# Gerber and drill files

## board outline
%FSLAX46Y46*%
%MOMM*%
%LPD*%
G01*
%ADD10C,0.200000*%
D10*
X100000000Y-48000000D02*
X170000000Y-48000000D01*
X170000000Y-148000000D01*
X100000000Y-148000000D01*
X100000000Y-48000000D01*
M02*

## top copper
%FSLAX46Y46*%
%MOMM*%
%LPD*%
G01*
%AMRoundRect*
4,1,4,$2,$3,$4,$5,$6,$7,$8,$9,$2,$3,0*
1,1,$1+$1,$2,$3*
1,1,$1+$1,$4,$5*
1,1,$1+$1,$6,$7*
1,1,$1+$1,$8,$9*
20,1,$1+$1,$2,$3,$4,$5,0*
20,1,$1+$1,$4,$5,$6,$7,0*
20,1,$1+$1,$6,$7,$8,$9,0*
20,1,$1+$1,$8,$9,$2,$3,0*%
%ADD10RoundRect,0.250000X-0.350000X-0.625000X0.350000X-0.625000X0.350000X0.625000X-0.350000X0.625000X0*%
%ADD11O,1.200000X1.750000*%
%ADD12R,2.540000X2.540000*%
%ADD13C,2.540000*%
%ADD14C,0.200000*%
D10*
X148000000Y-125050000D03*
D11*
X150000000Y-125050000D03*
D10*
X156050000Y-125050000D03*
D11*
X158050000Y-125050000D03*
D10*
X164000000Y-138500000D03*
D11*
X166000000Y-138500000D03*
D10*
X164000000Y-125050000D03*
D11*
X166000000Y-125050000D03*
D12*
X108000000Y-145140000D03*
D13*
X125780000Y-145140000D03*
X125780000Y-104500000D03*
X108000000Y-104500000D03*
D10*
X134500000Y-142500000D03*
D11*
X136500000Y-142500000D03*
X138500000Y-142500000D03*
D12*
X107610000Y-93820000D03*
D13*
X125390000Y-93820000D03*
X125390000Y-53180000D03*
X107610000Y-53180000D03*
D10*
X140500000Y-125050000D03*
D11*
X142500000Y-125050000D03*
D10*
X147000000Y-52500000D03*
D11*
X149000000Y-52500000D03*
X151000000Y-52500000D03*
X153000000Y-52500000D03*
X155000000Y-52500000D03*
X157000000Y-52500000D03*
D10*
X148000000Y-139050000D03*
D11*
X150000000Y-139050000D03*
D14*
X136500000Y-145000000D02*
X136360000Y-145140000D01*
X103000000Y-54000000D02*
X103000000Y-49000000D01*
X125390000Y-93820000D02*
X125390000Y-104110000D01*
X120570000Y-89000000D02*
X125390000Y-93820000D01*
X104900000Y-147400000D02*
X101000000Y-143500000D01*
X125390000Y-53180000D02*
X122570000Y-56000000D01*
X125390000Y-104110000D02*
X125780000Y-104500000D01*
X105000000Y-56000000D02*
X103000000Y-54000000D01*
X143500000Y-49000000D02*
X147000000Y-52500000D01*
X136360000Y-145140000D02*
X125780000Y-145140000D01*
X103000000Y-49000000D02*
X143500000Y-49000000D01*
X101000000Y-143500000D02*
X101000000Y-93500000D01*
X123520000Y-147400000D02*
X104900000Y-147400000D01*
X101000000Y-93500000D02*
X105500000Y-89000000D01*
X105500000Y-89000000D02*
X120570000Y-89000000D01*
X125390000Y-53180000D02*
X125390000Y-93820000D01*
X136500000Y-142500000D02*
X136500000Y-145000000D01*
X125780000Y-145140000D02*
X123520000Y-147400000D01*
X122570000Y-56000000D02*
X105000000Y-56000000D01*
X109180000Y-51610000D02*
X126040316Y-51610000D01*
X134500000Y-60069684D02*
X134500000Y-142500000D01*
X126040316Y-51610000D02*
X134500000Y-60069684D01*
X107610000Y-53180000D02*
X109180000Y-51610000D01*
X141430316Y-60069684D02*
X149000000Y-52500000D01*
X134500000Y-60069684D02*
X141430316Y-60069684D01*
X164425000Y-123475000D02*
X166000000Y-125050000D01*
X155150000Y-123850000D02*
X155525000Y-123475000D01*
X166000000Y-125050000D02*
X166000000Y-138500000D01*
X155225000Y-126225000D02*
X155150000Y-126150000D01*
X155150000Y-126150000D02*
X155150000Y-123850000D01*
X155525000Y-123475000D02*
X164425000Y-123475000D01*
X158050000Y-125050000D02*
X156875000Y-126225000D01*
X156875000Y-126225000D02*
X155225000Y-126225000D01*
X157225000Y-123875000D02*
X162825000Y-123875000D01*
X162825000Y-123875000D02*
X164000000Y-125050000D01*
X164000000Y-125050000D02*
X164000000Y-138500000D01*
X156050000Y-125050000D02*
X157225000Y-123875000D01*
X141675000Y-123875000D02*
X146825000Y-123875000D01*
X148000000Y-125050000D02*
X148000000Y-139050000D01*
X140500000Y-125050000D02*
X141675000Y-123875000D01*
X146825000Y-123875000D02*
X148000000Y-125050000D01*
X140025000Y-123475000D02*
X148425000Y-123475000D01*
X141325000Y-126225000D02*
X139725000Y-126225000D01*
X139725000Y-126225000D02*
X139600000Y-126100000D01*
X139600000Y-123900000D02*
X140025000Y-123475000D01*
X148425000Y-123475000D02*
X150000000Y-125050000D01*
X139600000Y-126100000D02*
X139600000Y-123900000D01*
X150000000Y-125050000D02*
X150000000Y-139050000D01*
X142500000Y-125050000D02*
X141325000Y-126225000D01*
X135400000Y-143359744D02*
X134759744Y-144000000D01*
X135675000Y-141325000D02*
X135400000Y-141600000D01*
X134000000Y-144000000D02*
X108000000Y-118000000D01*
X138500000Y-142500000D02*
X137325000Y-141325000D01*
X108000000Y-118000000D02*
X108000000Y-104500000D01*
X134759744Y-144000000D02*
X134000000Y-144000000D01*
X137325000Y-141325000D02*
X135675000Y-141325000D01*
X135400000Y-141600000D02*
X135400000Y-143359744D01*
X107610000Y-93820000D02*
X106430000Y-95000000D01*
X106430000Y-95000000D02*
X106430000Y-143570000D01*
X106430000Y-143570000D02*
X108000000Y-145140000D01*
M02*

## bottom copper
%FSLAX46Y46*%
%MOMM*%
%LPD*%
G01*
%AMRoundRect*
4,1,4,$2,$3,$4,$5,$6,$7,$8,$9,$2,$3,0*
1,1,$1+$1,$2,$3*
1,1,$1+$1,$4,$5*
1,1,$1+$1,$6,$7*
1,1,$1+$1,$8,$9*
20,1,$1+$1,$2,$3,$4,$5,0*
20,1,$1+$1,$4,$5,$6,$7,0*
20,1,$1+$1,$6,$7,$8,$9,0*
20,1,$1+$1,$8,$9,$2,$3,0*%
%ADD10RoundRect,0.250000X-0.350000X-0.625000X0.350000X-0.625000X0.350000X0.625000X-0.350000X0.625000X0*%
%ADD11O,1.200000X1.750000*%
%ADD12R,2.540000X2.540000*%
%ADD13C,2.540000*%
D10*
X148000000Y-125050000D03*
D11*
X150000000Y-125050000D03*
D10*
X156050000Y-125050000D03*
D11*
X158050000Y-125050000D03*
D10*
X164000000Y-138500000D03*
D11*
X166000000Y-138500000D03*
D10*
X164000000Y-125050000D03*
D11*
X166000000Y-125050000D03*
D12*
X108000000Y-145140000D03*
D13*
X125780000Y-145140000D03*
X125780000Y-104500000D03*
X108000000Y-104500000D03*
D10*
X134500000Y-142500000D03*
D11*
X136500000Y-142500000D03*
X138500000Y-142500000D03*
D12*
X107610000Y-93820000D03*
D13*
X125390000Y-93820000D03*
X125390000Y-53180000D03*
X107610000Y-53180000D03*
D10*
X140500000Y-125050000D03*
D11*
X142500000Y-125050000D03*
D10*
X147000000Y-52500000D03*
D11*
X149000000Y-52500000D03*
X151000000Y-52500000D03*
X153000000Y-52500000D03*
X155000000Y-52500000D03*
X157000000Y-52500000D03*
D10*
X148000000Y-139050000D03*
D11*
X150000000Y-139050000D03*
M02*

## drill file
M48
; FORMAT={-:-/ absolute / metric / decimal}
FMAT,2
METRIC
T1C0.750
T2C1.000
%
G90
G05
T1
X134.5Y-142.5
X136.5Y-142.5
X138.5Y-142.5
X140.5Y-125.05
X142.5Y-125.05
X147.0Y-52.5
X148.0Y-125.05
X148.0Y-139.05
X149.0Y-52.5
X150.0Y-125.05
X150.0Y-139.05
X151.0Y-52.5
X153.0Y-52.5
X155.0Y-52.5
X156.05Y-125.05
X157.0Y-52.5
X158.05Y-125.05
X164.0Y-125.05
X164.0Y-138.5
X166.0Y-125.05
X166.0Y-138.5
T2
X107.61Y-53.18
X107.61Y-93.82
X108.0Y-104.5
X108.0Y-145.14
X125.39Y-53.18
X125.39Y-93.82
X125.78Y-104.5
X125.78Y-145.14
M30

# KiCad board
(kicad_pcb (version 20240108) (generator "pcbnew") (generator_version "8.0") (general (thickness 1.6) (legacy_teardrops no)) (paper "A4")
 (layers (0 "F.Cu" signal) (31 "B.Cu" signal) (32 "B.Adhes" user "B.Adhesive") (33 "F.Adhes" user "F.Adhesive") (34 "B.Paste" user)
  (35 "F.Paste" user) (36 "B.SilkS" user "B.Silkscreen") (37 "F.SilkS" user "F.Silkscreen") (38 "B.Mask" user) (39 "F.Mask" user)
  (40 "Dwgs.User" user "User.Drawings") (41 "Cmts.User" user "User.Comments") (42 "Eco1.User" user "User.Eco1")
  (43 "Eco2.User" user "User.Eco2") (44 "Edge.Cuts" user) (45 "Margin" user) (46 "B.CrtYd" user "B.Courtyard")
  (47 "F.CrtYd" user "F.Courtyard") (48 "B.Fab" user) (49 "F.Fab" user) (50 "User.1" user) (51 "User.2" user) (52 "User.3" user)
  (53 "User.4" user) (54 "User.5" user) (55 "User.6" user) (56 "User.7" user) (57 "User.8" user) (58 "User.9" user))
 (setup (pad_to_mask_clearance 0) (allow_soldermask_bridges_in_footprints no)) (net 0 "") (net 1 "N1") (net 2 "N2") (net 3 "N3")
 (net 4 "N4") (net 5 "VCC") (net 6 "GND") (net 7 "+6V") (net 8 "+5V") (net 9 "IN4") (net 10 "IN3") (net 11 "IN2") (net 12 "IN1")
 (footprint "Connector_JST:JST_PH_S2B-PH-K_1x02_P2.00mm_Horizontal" (layer "F.Cu") (at 148 125.05)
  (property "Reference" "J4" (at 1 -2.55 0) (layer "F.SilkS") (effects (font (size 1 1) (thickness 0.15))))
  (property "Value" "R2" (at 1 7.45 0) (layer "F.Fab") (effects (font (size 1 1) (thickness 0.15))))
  (pad "1" thru_hole roundrect (at 0 0) (size 1.2 1.75) (drill 0.75) (layers "*.Cu" "*.Mask") (remove_unused_layers no)
   (roundrect_rratio 0.208333) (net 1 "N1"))
  (pad "2" thru_hole oval (at 2 0) (size 1.2 1.75) (drill 0.75) (layers "*.Cu" "*.Mask") (remove_unused_layers no) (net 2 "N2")))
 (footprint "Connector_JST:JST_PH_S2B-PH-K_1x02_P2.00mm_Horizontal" (layer "F.Cu") (at 156.05 125.05)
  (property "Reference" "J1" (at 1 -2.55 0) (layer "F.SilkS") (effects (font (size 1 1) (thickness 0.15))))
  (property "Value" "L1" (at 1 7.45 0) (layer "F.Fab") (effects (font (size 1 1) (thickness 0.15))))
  (pad "1" thru_hole roundrect (at 0 0) (size 1.2 1.75) (drill 0.75) (layers "*.Cu" "*.Mask") (remove_unused_layers no)
   (roundrect_rratio 0.208333) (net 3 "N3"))
  (pad "2" thru_hole oval (at 2 0) (size 1.2 1.75) (drill 0.75) (layers "*.Cu" "*.Mask") (remove_unused_layers no) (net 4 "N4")))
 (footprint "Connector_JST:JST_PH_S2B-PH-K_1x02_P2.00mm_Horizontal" (layer "F.Cu") (at 164 138.5)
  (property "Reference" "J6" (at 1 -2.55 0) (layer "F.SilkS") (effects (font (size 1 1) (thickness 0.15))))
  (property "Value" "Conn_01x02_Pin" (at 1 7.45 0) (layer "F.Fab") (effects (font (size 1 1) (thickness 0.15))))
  (pad "1" thru_hole roundrect (at 0 0) (size 1.2 1.75) (drill 0.75) (layers "*.Cu" "*.Mask") (remove_unused_layers no)
   (roundrect_rratio 0.208333) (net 3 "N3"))
  (pad "2" thru_hole oval (at 2 0) (size 1.2 1.75) (drill 0.75) (layers "*.Cu" "*.Mask") (remove_unused_layers no) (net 4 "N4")))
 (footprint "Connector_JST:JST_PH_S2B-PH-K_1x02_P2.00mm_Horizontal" (layer "F.Cu") (at 164 125.05)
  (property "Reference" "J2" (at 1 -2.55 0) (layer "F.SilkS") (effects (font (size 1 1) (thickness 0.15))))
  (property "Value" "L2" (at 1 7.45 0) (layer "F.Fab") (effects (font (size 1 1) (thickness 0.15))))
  (pad "1" thru_hole roundrect (at 0 0) (size 1.2 1.75) (drill 0.75) (layers "*.Cu" "*.Mask") (remove_unused_layers no)
   (roundrect_rratio 0.208333) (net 3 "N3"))
  (pad "2" thru_hole oval (at 2 0) (size 1.2 1.75) (drill 0.75) (layers "*.Cu" "*.Mask") (remove_unused_layers no) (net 4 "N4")))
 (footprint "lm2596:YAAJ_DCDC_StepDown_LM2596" (layer "F.Cu") (at 108 145.14 90)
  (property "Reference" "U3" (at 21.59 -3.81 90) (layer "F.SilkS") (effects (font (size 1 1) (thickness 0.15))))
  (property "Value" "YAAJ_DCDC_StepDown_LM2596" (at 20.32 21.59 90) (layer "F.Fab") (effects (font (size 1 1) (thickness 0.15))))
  (pad "1" thru_hole rect (at 0 0 90) (size 2.54 2.54) (drill 1) (layers "*.Cu" "*.Mask") (remove_unused_layers no) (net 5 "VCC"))
  (pad "2" thru_hole circle (at 0 17.78 90) (size 2.54 2.54) (drill 1) (layers "*.Cu" "*.Mask") (remove_unused_layers no) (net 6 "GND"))
  (pad "3" thru_hole circle (at 40.64 17.78 90) (size 2.54 2.54) (drill 1) (layers "*.Cu" "*.Mask") (remove_unused_layers no) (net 6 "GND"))
  (pad "4" thru_hole circle (at 40.64 0 90) (size 2.54 2.54) (drill 1) (layers "*.Cu" "*.Mask") (remove_unused_layers no) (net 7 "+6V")))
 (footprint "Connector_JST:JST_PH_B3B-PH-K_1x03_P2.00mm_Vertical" (layer "F.Cu") (at 134.5 142.5)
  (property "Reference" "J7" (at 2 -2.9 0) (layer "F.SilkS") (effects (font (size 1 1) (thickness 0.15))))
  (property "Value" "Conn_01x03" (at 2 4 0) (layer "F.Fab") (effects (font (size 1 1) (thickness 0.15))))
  (pad "1" thru_hole roundrect (at 0 0) (size 1.2 1.75) (drill 0.75) (layers "*.Cu" "*.Mask") (remove_unused_layers no)
   (roundrect_rratio 0.208333) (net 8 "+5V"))
  (pad "2" thru_hole oval (at 2 0) (size 1.2 1.75) (drill 0.75) (layers "*.Cu" "*.Mask") (remove_unused_layers no) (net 6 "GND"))
  (pad "3" thru_hole oval (at 4 0) (size 1.2 1.75) (drill 0.75) (layers "*.Cu" "*.Mask") (remove_unused_layers no) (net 7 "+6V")))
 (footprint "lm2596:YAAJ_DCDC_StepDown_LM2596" (layer "F.Cu") (at 107.61 93.82 90)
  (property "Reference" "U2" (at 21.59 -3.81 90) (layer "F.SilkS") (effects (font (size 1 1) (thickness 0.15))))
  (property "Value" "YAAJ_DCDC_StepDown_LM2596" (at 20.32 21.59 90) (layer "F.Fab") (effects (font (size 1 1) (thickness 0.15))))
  (pad "1" thru_hole rect (at 0 0 90) (size 2.54 2.54) (drill 1) (layers "*.Cu" "*.Mask") (remove_unused_layers no) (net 5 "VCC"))
  (pad "2" thru_hole circle (at 0 17.78 90) (size 2.54 2.54) (drill 1) (layers "*.Cu" "*.Mask") (remove_unused_layers no) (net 6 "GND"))
  (pad "3" thru_hole circle (at 40.64 17.78 90) (size 2.54 2.54) (drill 1) (layers "*.Cu" "*.Mask") (remove_unused_layers no) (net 6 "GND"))
  (pad "4" thru_hole circle (at 40.64 0 90) (size 2.54 2.54) (drill 1) (layers "*.Cu" "*.Mask") (remove_unused_layers no) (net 8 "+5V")))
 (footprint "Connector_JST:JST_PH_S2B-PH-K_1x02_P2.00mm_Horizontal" (layer "F.Cu") (at 140.5 125.05)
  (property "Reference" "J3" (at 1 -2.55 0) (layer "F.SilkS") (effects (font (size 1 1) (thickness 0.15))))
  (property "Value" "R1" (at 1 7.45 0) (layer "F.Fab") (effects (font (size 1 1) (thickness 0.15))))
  (pad "1" thru_hole roundrect (at 0 0) (size 1.2 1.75) (drill 0.75) (layers "*.Cu" "*.Mask") (remove_unused_layers no)
   (roundrect_rratio 0.208333) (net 1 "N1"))
  (pad "2" thru_hole oval (at 2 0) (size 1.2 1.75) (drill 0.75) (layers "*.Cu" "*.Mask") (remove_unused_layers no) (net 2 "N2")))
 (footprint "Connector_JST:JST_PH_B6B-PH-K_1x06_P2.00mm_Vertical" (layer "F.Cu") (at 147 52.5)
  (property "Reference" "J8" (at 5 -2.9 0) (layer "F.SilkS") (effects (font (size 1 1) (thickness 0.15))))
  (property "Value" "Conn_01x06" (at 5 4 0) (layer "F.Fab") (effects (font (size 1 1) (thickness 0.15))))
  (pad "1" thru_hole roundrect (at 0 0) (size 1.2 1.75) (drill 0.75) (layers "*.Cu" "*.Mask") (remove_unused_layers no)
   (roundrect_rratio 0.208333) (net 6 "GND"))
  (pad "2" thru_hole oval (at 2 0) (size 1.2 1.75) (drill 0.75) (layers "*.Cu" "*.Mask") (remove_unused_layers no) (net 8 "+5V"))
  (pad "3" thru_hole oval (at 4 0) (size 1.2 1.75) (drill 0.75) (layers "*.Cu" "*.Mask") (remove_unused_layers no) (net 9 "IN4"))
  (pad "4" thru_hole oval (at 6 0) (size 1.2 1.75) (drill 0.75) (layers "*.Cu" "*.Mask") (remove_unused_layers no) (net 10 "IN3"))
  (pad "5" thru_hole oval (at 8 0) (size 1.2 1.75) (drill 0.75) (layers "*.Cu" "*.Mask") (remove_unused_layers no) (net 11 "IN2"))
  (pad "6" thru_hole oval (at 10 0) (size 1.2 1.75) (drill 0.75) (layers "*.Cu" "*.Mask") (remove_unused_layers no) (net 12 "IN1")))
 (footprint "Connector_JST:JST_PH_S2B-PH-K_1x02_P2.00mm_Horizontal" (layer "F.Cu") (at 148 139.05)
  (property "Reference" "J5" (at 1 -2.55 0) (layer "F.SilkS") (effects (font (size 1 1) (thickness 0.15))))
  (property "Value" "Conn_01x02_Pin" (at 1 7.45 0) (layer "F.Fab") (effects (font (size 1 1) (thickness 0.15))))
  (pad "1" thru_hole roundrect (at 0 0) (size 1.2 1.75) (drill 0.75) (layers "*.Cu" "*.Mask") (remove_unused_layers no)
   (roundrect_rratio 0.208333) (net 1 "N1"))
  (pad "2" thru_hole oval (at 2 0) (size 1.2 1.75) (drill 0.75) (layers "*.Cu" "*.Mask") (remove_unused_layers no) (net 2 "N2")))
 (gr_rect (start 100 48) (end 170 148) (stroke (width 0.2) (type default)) (fill none) (layer "Edge.Cuts"))
 (segment (start 136.5 145) (end 136.36 145.14) (width 0.2) (layer "F.Cu") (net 6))
 (segment (start 103 54) (end 103 49) (width 0.2) (layer "F.Cu") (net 6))
 (segment (start 125.39 93.82) (end 125.39 104.11) (width 0.2) (layer "F.Cu") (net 6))
 (segment (start 120.57 89) (end 125.39 93.82) (width 0.2) (layer "F.Cu") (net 6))
 (segment (start 104.9 147.4) (end 101 143.5) (width 0.2) (layer "F.Cu") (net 6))
 (segment (start 125.39 53.18) (end 122.57 56) (width 0.2) (layer "F.Cu") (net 6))
 (segment (start 125.39 104.11) (end 125.78 104.5) (width 0.2) (layer "F.Cu") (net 6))
 (segment (start 105 56) (end 103 54) (width 0.2) (layer "F.Cu") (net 6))
 (segment (start 143.5 49) (end 147 52.5) (width 0.2) (layer "F.Cu") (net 6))
 (segment (start 136.36 145.14) (end 125.78 145.14) (width 0.2) (layer "F.Cu") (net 6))
 (segment (start 103 49) (end 143.5 49) (width 0.2) (layer "F.Cu") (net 6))
 (segment (start 101 143.5) (end 101 93.5) (width 0.2) (layer "F.Cu") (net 6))
 (segment (start 123.52 147.4) (end 104.9 147.4) (width 0.2) (layer "F.Cu") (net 6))
 (segment (start 101 93.5) (end 105.5 89) (width 0.2) (layer "F.Cu") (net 6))
 (segment (start 105.5 89) (end 120.57 89) (width 0.2) (layer "F.Cu") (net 6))
 (segment (start 125.39 53.18) (end 125.39 93.82) (width 0.2) (layer "F.Cu") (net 6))
 (segment (start 136.5 142.5) (end 136.5 145) (width 0.2) (layer "F.Cu") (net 6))
 (segment (start 125.78 145.14) (end 123.52 147.4) (width 0.2) (layer "F.Cu") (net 6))
 (segment (start 122.57 56) (end 105 56) (width 0.2) (layer "F.Cu") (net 6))
 (segment (start 109.18 51.61) (end 126.040316 51.61) (width 0.2) (layer "F.Cu") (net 8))
 (segment (start 134.5 60.069684) (end 134.5 142.5) (width 0.2) (layer "F.Cu") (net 8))
 (segment (start 126.040316 51.61) (end 134.5 60.069684) (width 0.2) (layer "F.Cu") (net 8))
 (segment (start 107.61 53.18) (end 109.18 51.61) (width 0.2) (layer "F.Cu") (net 8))
 (segment (start 141.430316 60.069684) (end 149 52.5) (width 0.2) (layer "F.Cu") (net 8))
 (segment (start 134.5 60.069684) (end 141.430316 60.069684) (width 0.2) (layer "F.Cu") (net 8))
 (segment (start 164.425 123.475) (end 166 125.05) (width 0.2) (layer "F.Cu") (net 4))
 (segment (start 155.15 123.85) (end 155.525 123.475) (width 0.2) (layer "F.Cu") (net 4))
 (segment (start 166 125.05) (end 166 138.5) (width 0.2) (layer "F.Cu") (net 4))
 (segment (start 155.225 126.225) (end 155.15 126.15) (width 0.2) (layer "F.Cu") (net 4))
 (segment (start 155.15 126.15) (end 155.15 123.85) (width 0.2) (layer "F.Cu") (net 4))
 (segment (start 155.525 123.475) (end 164.425 123.475) (width 0.2) (layer "F.Cu") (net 4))
 (segment (start 158.05 125.05) (end 156.875 126.225) (width 0.2) (layer "F.Cu") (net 4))
 (segment (start 156.875 126.225) (end 155.225 126.225) (width 0.2) (layer "F.Cu") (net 4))
 (segment (start 157.225 123.875) (end 162.825 123.875) (width 0.2) (layer "F.Cu") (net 3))
 (segment (start 162.825 123.875) (end 164 125.05) (width 0.2) (layer "F.Cu") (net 3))
 (segment (start 164 125.05) (end 164 138.5) (width 0.2) (layer "F.Cu") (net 3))
 (segment (start 156.05 125.05) (end 157.225 123.875) (width 0.2) (layer "F.Cu") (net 3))
 (segment (start 141.675 123.875) (end 146.825 123.875) (width 0.2) (layer "F.Cu") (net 1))
 (segment (start 148 125.05) (end 148 139.05) (width 0.2) (layer "F.Cu") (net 1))
 (segment (start 140.5 125.05) (end 141.675 123.875) (width 0.2) (layer "F.Cu") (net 1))
 (segment (start 146.825 123.875) (end 148 125.05) (width 0.2) (layer "F.Cu") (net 1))
 (segment (start 140.025 123.475) (end 148.425 123.475) (width 0.2) (layer "F.Cu") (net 2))
 (segment (start 141.325 126.225) (end 139.725 126.225) (width 0.2) (layer "F.Cu") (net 2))
 (segment (start 139.725 126.225) (end 139.6 126.1) (width 0.2) (layer "F.Cu") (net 2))
 (segment (start 139.6 123.9) (end 140.025 123.475) (width 0.2) (layer "F.Cu") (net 2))
 (segment (start 148.425 123.475) (end 150 125.05) (width 0.2) (layer "F.Cu") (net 2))
 (segment (start 139.6 126.1) (end 139.6 123.9) (width 0.2) (layer "F.Cu") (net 2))
 (segment (start 150 125.05) (end 150 139.05) (width 0.2) (layer "F.Cu") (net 2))
 (segment (start 142.5 125.05) (end 141.325 126.225) (width 0.2) (layer "F.Cu") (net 2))
 (segment (start 135.4 143.359744) (end 134.759744 144) (width 0.2) (layer "F.Cu") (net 7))
 (segment (start 135.675 141.325) (end 135.4 141.6) (width 0.2) (layer "F.Cu") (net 7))
 (segment (start 134 144) (end 108 118) (width 0.2) (layer "F.Cu") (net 7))
 (segment (start 138.5 142.5) (end 137.325 141.325) (width 0.2) (layer "F.Cu") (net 7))
 (segment (start 108 118) (end 108 104.5) (width 0.2) (layer "F.Cu") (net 7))
 (segment (start 134.759744 144) (end 134 144) (width 0.2) (layer "F.Cu") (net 7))
 (segment (start 137.325 141.325) (end 135.675 141.325) (width 0.2) (layer "F.Cu") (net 7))
 (segment (start 135.4 141.6) (end 135.4 143.359744) (width 0.2) (layer "F.Cu") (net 7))
 (segment (start 107.61 93.82) (end 106.43 95) (width 0.2) (layer "F.Cu") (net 5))
 (segment (start 106.43 95) (end 106.43 143.57) (width 0.2) (layer "F.Cu") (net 5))
 (segment (start 106.43 143.57) (end 108 145.14) (width 0.2) (layer "F.Cu") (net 5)))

